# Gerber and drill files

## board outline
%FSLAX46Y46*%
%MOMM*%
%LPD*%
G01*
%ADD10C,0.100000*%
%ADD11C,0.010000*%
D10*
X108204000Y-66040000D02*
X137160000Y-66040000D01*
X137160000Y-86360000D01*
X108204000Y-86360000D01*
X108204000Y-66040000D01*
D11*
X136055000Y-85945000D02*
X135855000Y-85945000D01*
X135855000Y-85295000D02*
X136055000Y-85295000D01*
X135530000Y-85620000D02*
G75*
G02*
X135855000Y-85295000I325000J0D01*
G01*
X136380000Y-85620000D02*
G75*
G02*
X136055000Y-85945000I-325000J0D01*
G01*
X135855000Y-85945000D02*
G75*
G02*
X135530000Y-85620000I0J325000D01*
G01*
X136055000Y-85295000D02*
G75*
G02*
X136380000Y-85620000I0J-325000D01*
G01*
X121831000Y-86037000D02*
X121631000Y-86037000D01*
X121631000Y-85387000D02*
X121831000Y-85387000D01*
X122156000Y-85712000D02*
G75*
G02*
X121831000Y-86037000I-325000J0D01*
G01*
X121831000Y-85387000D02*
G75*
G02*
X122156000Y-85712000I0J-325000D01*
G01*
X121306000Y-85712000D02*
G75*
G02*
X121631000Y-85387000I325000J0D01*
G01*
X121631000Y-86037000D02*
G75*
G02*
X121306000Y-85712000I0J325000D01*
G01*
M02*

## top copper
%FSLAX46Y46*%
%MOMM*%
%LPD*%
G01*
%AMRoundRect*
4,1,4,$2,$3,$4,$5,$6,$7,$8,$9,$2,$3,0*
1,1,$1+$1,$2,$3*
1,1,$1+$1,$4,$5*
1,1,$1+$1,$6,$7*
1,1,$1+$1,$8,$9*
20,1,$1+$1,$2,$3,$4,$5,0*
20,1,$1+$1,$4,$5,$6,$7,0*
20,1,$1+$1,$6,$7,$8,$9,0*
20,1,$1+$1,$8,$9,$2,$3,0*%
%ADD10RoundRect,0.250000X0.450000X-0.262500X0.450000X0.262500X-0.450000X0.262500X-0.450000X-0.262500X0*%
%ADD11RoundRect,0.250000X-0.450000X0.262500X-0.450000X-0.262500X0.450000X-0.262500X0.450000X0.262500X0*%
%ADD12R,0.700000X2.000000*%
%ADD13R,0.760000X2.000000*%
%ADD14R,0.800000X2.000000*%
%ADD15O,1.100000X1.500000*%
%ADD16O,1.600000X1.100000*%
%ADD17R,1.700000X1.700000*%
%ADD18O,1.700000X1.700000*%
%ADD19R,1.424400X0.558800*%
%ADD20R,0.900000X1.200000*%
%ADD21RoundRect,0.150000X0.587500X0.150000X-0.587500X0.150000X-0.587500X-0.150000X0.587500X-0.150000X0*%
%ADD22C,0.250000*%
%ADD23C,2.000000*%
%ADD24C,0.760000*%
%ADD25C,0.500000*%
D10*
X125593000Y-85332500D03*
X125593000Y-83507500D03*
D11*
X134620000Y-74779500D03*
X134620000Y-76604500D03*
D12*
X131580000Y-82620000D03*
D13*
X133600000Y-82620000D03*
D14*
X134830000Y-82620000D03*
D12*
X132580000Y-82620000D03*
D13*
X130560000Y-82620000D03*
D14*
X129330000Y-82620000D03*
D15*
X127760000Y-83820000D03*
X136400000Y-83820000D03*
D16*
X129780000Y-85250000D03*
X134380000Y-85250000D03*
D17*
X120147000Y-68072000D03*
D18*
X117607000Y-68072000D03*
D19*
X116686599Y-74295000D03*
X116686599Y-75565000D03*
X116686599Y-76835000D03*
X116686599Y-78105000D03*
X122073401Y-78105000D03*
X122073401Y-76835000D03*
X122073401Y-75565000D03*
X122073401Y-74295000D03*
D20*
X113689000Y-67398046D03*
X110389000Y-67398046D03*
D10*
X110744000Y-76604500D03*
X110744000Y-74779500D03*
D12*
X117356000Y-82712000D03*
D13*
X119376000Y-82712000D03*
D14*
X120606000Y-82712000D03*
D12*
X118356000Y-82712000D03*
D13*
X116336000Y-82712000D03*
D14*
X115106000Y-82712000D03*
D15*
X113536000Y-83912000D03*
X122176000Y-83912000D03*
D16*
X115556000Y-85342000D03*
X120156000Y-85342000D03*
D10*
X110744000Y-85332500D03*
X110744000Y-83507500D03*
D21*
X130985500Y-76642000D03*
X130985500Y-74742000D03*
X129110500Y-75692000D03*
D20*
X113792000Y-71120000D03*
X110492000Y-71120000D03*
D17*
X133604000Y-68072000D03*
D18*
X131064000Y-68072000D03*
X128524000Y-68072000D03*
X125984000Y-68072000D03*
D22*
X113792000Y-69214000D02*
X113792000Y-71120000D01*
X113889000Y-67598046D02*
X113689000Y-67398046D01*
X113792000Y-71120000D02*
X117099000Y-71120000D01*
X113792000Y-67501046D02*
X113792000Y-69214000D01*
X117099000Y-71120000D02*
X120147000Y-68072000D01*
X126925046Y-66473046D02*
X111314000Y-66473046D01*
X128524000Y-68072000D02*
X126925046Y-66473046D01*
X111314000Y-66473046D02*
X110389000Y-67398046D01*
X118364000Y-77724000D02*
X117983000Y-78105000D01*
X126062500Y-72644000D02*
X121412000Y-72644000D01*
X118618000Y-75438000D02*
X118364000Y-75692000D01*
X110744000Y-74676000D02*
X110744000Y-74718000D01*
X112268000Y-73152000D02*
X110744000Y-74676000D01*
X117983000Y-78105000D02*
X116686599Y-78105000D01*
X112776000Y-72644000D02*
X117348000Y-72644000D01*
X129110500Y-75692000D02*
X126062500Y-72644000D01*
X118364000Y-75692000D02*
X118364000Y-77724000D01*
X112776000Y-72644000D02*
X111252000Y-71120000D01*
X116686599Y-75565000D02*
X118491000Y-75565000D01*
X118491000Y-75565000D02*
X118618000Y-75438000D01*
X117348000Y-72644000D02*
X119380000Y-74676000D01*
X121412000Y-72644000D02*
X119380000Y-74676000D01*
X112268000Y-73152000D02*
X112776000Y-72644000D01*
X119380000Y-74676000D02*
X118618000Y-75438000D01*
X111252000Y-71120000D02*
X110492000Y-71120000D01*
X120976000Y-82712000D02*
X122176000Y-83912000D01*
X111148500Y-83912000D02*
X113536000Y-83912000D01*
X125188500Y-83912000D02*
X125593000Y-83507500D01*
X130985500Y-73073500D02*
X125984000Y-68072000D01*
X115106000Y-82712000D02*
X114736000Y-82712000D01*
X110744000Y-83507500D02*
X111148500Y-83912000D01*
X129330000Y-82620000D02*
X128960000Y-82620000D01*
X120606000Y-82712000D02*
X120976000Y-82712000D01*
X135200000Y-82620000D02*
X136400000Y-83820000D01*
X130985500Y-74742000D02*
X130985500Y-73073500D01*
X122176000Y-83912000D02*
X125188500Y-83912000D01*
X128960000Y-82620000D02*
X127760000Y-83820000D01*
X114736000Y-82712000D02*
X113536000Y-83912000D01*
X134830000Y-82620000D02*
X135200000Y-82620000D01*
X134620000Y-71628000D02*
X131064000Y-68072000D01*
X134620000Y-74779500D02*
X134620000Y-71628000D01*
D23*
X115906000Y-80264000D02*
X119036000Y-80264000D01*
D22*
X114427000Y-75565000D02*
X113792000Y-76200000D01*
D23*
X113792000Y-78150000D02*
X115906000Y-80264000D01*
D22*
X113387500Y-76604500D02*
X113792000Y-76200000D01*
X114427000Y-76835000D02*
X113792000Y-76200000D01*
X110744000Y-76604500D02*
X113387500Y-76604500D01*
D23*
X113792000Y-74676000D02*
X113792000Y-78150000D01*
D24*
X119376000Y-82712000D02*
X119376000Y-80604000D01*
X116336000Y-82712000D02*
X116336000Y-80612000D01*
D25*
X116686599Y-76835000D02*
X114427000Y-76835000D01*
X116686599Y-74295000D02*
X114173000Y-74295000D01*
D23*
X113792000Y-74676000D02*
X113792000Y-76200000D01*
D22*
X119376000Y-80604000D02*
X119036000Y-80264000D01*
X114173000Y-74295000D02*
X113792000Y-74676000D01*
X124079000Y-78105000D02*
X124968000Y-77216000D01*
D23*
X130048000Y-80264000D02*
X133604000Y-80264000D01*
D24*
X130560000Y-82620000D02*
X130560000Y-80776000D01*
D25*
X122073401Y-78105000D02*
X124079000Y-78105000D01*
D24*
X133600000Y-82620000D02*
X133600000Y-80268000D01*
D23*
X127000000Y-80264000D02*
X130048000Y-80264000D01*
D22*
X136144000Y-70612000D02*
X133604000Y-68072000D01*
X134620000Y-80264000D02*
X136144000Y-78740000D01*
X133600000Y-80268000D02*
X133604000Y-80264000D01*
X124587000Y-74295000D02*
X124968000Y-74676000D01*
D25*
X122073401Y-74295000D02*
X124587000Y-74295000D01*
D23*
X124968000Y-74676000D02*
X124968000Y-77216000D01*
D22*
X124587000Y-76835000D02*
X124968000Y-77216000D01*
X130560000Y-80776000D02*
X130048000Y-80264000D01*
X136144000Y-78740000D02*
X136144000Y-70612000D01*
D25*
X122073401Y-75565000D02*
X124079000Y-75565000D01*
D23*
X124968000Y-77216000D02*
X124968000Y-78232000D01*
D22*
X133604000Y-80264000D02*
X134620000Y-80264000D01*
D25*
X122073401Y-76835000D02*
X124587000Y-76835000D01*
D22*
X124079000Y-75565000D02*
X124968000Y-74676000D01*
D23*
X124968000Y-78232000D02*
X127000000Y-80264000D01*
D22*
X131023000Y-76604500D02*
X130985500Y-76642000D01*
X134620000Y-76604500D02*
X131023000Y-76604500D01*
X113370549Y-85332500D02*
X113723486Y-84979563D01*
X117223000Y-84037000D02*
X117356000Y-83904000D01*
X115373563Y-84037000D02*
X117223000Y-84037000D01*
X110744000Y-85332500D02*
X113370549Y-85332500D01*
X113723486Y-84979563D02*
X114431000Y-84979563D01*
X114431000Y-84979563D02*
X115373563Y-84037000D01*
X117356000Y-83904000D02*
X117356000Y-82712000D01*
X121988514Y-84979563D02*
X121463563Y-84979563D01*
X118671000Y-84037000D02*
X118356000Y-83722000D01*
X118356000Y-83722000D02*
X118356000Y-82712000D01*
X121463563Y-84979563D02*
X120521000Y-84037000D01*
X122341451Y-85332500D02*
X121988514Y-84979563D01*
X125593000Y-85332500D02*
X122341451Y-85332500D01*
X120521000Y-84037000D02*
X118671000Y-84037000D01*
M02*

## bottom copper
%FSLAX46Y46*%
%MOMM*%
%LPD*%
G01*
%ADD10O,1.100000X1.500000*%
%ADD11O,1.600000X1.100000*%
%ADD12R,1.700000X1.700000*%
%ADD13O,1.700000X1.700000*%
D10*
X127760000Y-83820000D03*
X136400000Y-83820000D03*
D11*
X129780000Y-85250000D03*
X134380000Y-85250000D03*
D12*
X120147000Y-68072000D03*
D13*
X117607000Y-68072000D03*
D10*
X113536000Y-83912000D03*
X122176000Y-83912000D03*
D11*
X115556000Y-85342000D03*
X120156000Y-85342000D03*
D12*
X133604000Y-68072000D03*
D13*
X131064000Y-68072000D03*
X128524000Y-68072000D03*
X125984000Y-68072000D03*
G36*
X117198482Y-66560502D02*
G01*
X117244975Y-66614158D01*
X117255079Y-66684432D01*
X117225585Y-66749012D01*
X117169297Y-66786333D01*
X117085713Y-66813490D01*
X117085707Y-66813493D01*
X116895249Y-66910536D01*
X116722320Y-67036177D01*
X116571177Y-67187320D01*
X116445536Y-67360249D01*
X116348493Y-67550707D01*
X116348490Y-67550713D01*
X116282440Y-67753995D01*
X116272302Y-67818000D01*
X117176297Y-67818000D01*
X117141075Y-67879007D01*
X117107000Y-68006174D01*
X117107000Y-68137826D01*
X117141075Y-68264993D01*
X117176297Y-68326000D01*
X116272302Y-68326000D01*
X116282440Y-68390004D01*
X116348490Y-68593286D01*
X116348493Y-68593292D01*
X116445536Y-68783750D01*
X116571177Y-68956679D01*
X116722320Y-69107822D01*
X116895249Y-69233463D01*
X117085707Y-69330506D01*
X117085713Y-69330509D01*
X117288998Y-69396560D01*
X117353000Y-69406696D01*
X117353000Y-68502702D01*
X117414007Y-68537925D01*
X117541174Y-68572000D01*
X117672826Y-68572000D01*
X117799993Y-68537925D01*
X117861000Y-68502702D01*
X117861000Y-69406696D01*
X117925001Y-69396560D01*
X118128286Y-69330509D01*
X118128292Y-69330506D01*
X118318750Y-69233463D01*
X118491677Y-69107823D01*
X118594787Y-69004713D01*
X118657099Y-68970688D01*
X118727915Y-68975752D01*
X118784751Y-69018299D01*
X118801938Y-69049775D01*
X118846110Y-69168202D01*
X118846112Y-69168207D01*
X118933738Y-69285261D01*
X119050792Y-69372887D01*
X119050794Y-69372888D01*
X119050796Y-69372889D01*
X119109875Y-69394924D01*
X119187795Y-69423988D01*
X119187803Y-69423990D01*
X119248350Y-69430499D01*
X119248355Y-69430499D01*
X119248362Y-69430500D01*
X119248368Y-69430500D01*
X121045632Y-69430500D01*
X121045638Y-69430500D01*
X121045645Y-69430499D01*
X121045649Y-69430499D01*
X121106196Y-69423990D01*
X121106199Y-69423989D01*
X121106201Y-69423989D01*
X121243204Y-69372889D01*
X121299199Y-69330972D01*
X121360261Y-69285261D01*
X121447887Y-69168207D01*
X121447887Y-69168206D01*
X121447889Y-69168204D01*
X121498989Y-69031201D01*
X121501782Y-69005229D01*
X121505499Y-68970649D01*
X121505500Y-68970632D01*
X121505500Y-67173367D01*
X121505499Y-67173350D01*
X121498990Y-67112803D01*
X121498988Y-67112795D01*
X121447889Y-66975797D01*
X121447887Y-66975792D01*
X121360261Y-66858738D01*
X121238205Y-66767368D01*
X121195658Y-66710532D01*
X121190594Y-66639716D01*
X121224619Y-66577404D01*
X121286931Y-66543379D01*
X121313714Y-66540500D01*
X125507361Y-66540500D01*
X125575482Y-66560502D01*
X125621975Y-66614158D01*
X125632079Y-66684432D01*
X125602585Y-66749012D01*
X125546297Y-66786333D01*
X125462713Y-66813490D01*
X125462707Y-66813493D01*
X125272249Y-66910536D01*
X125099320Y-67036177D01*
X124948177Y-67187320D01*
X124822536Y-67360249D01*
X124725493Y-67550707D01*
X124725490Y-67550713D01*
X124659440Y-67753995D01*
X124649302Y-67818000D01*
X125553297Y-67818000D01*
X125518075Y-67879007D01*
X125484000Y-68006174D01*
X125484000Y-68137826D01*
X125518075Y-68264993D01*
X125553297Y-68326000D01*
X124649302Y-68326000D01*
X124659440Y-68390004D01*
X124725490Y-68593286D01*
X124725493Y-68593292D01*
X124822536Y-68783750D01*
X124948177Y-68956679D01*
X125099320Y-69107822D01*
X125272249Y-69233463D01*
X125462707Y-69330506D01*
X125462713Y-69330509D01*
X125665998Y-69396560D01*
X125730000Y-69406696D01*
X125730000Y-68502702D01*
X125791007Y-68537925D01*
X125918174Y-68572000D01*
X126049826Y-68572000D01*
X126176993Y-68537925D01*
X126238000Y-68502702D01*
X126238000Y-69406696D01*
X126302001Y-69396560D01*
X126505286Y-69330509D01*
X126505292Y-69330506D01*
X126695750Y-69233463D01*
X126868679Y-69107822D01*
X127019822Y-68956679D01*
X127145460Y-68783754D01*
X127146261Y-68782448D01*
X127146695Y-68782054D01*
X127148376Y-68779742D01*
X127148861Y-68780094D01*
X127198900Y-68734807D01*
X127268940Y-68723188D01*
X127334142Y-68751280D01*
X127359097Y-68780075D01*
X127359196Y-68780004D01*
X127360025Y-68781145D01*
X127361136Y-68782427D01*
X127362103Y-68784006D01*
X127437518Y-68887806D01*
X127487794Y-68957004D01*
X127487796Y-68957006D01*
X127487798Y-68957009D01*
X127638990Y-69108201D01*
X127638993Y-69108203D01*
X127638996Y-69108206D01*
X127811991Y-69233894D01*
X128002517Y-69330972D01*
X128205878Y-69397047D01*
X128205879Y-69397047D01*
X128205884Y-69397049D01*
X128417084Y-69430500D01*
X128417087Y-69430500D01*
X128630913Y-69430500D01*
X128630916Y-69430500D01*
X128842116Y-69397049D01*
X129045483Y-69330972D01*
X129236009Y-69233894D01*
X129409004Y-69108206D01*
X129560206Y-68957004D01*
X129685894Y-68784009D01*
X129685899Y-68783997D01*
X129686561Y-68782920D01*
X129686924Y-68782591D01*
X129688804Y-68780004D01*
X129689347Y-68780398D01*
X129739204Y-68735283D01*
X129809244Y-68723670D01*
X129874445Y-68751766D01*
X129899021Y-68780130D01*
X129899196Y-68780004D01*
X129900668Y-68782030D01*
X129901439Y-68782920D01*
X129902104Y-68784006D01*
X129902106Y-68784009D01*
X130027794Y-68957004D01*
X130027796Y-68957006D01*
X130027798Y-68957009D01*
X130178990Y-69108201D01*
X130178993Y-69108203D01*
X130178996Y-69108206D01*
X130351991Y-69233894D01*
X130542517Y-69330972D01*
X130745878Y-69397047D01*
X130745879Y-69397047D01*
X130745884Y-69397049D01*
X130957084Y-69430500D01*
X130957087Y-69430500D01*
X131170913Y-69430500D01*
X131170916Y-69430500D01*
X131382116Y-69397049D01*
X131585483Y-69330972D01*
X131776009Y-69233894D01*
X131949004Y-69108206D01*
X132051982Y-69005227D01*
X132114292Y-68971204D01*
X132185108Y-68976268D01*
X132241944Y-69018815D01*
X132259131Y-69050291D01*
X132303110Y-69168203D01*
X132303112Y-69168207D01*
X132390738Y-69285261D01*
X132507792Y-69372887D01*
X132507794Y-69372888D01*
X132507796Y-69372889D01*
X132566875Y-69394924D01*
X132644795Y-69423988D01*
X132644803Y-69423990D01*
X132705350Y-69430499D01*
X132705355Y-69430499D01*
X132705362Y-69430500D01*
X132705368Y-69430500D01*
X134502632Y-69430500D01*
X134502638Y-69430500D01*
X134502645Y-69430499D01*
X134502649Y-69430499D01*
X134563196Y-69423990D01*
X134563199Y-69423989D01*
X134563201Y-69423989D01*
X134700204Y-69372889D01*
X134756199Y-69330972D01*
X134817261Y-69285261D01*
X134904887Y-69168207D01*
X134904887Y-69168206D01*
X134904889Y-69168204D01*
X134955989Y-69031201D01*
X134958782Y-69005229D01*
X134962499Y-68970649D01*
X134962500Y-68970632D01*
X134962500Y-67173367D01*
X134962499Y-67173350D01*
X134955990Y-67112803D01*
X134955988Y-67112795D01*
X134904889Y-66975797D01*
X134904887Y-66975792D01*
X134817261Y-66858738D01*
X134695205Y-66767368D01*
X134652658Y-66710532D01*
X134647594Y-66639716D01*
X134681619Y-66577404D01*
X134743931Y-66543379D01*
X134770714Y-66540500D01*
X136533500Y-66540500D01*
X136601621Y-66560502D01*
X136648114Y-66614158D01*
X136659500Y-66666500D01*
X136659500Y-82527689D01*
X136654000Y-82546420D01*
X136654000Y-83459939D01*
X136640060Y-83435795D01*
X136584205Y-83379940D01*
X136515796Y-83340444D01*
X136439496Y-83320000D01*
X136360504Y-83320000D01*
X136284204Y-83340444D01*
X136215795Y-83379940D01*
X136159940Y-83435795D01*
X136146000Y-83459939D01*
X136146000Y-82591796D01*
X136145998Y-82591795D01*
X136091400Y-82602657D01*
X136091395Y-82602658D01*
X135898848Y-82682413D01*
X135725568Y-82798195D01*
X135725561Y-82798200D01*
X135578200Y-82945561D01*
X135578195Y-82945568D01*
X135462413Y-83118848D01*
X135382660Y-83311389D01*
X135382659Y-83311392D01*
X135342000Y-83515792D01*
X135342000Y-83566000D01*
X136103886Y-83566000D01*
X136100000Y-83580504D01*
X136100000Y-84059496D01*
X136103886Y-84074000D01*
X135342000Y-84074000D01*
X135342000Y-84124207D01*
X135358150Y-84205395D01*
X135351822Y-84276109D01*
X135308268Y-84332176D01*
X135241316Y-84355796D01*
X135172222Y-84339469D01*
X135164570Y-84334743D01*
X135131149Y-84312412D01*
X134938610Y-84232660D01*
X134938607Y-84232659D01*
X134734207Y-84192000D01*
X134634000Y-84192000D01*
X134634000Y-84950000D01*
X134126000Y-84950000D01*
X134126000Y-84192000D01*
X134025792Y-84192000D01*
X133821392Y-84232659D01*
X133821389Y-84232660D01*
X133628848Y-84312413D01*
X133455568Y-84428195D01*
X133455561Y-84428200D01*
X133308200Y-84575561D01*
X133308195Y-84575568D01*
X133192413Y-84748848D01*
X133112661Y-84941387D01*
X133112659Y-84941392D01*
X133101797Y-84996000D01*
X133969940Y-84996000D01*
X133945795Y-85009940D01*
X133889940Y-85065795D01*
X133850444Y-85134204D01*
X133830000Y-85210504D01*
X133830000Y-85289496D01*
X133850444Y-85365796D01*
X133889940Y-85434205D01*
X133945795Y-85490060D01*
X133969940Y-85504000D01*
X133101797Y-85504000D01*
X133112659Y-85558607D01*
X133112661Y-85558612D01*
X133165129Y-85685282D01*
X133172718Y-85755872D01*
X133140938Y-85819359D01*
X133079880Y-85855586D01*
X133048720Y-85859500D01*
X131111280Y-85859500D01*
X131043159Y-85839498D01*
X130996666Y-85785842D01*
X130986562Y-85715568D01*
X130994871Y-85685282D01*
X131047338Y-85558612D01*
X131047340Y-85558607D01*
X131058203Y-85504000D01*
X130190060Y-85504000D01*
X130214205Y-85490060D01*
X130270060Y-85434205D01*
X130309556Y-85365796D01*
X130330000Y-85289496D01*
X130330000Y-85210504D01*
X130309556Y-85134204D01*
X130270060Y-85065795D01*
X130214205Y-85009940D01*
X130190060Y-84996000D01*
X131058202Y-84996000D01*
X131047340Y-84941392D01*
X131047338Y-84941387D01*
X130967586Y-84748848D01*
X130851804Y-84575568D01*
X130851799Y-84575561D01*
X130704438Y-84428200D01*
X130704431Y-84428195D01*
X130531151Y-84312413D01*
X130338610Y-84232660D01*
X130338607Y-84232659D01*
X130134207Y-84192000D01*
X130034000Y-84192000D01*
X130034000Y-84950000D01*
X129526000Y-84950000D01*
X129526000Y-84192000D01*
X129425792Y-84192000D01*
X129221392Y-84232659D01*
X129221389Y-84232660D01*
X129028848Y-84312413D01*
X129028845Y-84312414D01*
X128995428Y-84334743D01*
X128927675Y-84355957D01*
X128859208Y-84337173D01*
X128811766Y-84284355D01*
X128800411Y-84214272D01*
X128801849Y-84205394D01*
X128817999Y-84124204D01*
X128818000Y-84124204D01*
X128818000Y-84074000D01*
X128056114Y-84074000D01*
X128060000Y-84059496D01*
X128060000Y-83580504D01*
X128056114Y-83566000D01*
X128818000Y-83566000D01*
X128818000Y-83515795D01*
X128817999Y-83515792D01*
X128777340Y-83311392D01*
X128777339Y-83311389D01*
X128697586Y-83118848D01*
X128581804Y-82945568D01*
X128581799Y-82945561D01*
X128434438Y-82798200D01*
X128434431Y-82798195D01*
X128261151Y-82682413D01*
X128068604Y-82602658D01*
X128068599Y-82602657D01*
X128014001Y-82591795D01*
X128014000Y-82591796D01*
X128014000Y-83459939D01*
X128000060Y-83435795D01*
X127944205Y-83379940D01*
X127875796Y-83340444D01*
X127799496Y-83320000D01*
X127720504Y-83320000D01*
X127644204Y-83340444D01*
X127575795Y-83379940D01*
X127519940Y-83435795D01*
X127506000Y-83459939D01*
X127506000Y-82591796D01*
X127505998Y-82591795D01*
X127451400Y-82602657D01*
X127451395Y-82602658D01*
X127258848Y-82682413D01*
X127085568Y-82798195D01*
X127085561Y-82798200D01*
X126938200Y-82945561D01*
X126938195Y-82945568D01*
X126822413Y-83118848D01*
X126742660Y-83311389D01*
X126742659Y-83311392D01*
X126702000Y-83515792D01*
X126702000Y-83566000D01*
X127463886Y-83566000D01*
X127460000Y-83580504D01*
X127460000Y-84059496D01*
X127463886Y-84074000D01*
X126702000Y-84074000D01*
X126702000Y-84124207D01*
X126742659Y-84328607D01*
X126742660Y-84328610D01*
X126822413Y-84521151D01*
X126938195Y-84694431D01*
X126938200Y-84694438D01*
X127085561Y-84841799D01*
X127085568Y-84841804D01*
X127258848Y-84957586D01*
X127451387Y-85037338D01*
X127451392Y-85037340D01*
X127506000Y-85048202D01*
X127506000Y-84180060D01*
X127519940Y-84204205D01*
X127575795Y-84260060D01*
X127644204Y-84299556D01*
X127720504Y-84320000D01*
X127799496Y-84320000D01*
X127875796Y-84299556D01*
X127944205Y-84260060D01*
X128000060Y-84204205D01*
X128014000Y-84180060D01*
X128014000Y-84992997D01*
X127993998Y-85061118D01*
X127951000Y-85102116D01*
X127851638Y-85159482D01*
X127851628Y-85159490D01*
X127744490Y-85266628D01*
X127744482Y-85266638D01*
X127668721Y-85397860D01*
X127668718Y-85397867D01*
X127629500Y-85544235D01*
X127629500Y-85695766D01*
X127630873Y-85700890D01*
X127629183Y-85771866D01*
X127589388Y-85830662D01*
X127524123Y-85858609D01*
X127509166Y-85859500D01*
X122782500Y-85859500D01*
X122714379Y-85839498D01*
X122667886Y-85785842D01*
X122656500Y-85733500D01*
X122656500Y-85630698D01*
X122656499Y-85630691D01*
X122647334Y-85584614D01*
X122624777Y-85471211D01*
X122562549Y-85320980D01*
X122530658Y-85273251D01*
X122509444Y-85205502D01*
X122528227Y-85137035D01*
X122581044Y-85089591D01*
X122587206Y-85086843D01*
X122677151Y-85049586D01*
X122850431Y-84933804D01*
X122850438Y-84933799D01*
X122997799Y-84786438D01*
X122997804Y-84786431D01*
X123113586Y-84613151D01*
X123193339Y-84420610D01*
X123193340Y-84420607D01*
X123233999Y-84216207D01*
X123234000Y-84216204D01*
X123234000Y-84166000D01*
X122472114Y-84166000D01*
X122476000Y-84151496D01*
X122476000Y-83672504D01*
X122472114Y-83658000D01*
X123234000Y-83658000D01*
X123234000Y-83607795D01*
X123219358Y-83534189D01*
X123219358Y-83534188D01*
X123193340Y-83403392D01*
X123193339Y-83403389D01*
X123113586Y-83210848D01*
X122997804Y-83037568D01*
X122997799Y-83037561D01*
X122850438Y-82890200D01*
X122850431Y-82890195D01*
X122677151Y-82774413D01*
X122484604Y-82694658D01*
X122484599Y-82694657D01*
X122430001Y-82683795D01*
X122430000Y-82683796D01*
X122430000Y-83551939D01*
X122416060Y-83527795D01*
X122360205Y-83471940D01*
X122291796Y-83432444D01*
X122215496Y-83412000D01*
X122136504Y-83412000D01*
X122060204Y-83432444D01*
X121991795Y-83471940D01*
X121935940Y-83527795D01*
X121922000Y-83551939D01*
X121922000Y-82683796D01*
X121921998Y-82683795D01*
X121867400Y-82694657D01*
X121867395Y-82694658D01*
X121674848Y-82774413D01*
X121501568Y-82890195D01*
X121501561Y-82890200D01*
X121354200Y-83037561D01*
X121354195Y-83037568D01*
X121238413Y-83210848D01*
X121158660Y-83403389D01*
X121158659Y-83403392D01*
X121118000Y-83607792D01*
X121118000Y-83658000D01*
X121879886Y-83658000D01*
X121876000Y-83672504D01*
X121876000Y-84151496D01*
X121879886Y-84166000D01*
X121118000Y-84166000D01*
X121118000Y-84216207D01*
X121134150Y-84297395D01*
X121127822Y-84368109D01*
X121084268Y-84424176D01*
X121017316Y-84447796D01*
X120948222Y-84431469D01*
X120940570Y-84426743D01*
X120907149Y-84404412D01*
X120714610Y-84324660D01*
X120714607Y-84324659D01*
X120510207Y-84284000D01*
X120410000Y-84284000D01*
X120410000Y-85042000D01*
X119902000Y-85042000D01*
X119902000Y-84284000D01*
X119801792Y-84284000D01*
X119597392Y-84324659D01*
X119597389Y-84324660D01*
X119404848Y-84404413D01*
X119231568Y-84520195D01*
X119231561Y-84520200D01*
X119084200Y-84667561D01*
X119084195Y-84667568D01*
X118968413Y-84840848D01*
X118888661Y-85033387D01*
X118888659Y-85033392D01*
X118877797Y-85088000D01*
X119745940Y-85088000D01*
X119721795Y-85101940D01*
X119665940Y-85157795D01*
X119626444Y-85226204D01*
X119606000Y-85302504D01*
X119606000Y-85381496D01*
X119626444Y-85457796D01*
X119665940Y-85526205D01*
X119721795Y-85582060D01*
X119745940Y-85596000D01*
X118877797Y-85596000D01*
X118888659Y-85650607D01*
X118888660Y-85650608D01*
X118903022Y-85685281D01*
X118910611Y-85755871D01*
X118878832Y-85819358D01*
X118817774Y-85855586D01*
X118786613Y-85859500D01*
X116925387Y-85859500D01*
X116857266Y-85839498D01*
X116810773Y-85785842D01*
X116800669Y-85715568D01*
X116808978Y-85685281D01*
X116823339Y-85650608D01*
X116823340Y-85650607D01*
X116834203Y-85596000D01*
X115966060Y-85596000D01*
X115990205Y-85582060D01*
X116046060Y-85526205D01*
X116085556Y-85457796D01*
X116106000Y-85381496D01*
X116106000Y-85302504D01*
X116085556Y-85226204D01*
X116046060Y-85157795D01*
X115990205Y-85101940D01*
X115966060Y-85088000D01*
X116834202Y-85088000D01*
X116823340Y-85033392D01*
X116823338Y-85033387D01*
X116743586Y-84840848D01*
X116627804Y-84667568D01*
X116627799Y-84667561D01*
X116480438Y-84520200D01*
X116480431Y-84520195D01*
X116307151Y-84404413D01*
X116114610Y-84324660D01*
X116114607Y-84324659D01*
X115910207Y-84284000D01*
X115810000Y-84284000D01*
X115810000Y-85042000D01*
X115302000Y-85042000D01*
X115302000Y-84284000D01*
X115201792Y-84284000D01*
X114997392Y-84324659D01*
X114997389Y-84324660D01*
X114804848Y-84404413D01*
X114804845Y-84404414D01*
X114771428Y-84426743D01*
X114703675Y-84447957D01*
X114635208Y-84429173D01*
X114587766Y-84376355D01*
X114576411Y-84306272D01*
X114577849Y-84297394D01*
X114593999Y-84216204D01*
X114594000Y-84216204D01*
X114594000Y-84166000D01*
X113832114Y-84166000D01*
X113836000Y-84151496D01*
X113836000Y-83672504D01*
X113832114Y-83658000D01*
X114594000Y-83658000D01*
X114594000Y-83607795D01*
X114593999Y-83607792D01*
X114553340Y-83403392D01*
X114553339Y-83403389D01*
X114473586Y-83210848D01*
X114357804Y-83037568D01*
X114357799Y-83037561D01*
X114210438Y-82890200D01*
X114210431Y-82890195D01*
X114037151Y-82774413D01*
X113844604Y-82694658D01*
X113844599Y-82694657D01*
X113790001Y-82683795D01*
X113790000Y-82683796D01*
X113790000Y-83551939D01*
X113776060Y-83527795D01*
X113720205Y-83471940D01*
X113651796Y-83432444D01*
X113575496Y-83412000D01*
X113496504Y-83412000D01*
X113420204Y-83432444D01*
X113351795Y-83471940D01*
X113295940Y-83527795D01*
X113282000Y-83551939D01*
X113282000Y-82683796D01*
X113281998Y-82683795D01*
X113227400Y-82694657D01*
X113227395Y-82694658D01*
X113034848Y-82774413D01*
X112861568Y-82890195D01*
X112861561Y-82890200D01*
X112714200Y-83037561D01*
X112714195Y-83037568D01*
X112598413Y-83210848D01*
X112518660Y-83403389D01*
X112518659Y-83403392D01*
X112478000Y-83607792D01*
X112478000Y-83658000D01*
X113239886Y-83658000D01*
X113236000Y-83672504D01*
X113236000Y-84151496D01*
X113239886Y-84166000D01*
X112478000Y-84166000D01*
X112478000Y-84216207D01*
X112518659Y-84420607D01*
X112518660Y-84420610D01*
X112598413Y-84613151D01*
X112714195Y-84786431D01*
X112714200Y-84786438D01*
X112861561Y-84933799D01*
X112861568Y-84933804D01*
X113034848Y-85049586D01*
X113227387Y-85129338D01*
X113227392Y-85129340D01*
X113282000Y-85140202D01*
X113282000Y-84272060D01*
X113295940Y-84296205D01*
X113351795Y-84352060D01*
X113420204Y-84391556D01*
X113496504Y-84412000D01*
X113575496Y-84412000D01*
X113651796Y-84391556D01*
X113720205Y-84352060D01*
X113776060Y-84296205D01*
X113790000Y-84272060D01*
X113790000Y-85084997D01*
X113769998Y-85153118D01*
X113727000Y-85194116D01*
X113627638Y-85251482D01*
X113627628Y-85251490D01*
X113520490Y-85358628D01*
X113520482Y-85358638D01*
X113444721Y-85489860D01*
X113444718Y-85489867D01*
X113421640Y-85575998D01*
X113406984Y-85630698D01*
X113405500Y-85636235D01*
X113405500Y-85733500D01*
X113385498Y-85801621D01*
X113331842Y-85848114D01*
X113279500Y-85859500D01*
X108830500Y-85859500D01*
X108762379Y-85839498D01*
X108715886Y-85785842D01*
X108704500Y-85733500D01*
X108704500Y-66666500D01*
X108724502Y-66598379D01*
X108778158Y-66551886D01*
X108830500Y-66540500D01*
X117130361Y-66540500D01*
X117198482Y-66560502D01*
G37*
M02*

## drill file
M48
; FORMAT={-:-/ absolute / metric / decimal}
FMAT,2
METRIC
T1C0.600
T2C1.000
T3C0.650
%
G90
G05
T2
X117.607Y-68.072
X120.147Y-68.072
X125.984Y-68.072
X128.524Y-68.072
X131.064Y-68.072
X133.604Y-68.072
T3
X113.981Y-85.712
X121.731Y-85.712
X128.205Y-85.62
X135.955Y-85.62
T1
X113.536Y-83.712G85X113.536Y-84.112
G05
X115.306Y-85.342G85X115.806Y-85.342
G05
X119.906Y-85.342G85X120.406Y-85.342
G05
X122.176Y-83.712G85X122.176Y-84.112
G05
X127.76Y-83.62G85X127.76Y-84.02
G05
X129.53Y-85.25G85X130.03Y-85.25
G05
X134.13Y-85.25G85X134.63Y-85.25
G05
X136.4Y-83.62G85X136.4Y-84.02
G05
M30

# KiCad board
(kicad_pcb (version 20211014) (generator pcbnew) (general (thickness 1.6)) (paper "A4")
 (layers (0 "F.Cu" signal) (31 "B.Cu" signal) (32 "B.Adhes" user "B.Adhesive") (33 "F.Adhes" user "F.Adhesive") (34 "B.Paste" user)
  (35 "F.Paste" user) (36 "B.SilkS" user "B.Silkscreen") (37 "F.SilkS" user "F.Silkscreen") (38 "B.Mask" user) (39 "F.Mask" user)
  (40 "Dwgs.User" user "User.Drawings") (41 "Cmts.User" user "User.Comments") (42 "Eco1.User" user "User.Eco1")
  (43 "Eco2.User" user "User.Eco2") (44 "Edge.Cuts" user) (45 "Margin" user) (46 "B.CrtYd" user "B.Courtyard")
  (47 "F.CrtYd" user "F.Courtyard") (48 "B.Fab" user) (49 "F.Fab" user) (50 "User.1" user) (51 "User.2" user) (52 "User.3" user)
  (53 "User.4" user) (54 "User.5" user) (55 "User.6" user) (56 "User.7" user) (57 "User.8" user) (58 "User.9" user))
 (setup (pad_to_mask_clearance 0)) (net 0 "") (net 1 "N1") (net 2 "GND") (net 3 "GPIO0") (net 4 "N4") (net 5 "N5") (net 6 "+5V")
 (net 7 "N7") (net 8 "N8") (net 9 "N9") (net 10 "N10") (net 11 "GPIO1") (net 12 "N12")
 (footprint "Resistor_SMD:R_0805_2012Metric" (layer "F.Cu") (at 125.593 84.42 90)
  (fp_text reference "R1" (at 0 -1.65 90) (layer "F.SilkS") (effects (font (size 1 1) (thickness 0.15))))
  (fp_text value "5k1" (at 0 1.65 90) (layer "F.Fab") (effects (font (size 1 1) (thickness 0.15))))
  (pad "1" smd roundrect (at -0.9125 0 90) (size 1.025 1.4) (layers "F.Cu" "F.Paste" "F.Mask") (roundrect_rratio 0.243902) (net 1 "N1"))
  (pad "2" smd roundrect (at 0.9125 0 90) (size 1.025 1.4) (layers "F.Cu" "F.Paste" "F.Mask") (roundrect_rratio 0.243902) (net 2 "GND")))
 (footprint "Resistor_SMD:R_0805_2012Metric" (layer "F.Cu") (at 134.62 75.692 -90)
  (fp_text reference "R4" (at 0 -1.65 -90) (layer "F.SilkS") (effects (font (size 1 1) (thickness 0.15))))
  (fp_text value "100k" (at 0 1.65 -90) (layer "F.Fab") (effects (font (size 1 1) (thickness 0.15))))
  (pad "1" smd roundrect (at -0.9125 0 270) (size 1.025 1.4) (layers "F.Cu" "F.Paste" "F.Mask") (roundrect_rratio 0.243902) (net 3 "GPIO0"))
  (pad "2" smd roundrect (at 0.9125 0 270) (size 1.025 1.4) (layers "F.Cu" "F.Paste" "F.Mask") (roundrect_rratio 0.243902) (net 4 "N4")))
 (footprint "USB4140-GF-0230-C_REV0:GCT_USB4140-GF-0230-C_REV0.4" (layer "F.Cu") (at 132.08 83.82)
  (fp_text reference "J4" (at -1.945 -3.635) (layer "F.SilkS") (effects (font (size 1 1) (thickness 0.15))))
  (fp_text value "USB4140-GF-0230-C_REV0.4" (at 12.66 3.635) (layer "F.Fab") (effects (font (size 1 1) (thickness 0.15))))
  (fp_line (start 3.975 2.125) (end 3.775 2.125) (layer "Edge.Cuts") (width 0.01))
  (fp_line (start 3.775 1.475) (end 3.975 1.475) (layer "Edge.Cuts") (width 0.01))
  (fp_arc (start 3.45 1.8) (mid 3.54519 1.57019) (end 3.775 1.475) (layer "Edge.Cuts") (width 0.01))
  (fp_arc (start 4.3 1.8) (mid 4.20481 2.02981) (end 3.975 2.125) (layer "Edge.Cuts") (width 0.01))
  (fp_arc (start 3.775 2.125) (mid 3.54519 2.02981) (end 3.45 1.8) (layer "Edge.Cuts") (width 0.01))
  (fp_arc (start 3.975 1.475) (mid 4.20481 1.57019) (end 4.3 1.8) (layer "Edge.Cuts") (width 0.01))
  (pad "" np_thru_hole circle locked (at 3.875 1.8) (size 0.65 0.65) (drill 0.65) (layers *.Cu *.Mask))
  (pad "" np_thru_hole circle locked (at -3.875 1.8) (size 0.65 0.65) (drill 0.65) (layers *.Cu *.Mask))
  (pad "A5" smd rect locked (at -0.5 -1.2) (size 0.7 2) (layers "F.Cu" "F.Paste" "F.Mask") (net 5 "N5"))
  (pad "A9" smd rect locked (at 1.52 -1.2) (size 0.76 2) (layers "F.Cu" "F.Paste" "F.Mask") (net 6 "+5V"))
  (pad "A12" smd rect locked (at 2.75 -1.2) (size 0.8 2) (layers "F.Cu" "F.Paste" "F.Mask") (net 2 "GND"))
  (pad "B5" smd rect locked (at 0.5 -1.2) (size 0.7 2) (layers "F.Cu" "F.Paste" "F.Mask") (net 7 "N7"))
  (pad "B9" smd rect locked (at -1.52 -1.2) (size 0.76 2) (layers "F.Cu" "F.Paste" "F.Mask") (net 6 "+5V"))
  (pad "B12" smd rect locked (at -2.75 -1.2) (size 0.8 2) (layers "F.Cu" "F.Paste" "F.Mask") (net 2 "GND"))
  (pad "S1" thru_hole oval locked (at -4.32 0) (size 1.1 1.5) (drill oval 0.6 1) (layers *.Cu *.Mask) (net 2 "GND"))
  (pad "S2" thru_hole oval locked (at 4.32 0) (size 1.1 1.5) (drill oval 0.6 1) (layers *.Cu *.Mask) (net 2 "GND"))
  (pad "S3" thru_hole oval locked (at -2.3 1.43) (size 1.6 1.1) (drill oval 1.1 0.6) (layers *.Cu *.Mask) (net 2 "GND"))
  (pad "S4" thru_hole oval locked (at 2.3 1.43) (size 1.6 1.1) (drill oval 1.1 0.6) (layers *.Cu *.Mask) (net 2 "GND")))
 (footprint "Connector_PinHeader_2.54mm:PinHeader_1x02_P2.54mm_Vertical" (layer "F.Cu") (at 120.147 68.072 -90)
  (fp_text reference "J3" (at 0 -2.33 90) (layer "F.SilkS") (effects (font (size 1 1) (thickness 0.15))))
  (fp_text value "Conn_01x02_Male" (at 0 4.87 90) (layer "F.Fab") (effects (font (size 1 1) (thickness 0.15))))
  (pad "1" thru_hole rect (at 0 0 270) (size 1.7 1.7) (drill 1) (layers *.Cu *.Mask) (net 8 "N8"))
  (pad "2" thru_hole oval (at 0 2.54 270) (size 1.7 1.7) (drill 1) (layers *.Cu *.Mask) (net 2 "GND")))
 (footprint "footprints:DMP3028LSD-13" (layer "F.Cu") (at 119.38 76.2)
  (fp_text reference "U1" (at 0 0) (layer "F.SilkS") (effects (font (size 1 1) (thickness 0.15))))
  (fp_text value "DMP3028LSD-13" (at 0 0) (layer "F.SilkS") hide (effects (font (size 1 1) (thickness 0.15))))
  (pad "1" smd rect (at -2.693401 -1.905) (size 1.4244 0.5588) (layers "F.Cu" "F.Paste" "F.Mask") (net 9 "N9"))
  (pad "2" smd rect (at -2.693401 -0.635) (size 1.4244 0.5588) (layers "F.Cu" "F.Paste" "F.Mask") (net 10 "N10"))
  (pad "3" smd rect (at -2.693401 0.635) (size 1.4244 0.5588) (layers "F.Cu" "F.Paste" "F.Mask") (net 9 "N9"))
  (pad "4" smd rect (at -2.693401 1.905) (size 1.4244 0.5588) (layers "F.Cu" "F.Paste" "F.Mask") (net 10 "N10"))
  (pad "5" smd rect (at 2.693401 1.905) (size 1.4244 0.5588) (layers "F.Cu" "F.Paste" "F.Mask") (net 6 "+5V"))
  (pad "6" smd rect (at 2.693401 0.635) (size 1.4244 0.5588) (layers "F.Cu" "F.Paste" "F.Mask") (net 6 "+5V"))
  (pad "7" smd rect (at 2.693401 -0.635) (size 1.4244 0.5588) (layers "F.Cu" "F.Paste" "F.Mask") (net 6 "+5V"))
  (pad "8" smd rect (at 2.693401 -1.905) (size 1.4244 0.5588) (layers "F.Cu" "F.Paste" "F.Mask") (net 6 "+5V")))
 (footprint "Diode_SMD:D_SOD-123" (layer "F.Cu") (at 112.039 67.398046 180)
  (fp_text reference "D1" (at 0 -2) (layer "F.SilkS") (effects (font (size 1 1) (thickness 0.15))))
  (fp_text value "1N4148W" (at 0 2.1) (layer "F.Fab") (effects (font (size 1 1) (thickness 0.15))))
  (pad "1" smd rect (at -1.65 0 180) (size 0.9 1.2) (layers "F.Cu" "F.Paste" "F.Mask") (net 8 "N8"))
  (pad "2" smd rect (at 1.65 0 180) (size 0.9 1.2) (layers "F.Cu" "F.Paste" "F.Mask") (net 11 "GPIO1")))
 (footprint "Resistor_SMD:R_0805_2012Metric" (layer "F.Cu") (at 110.744 75.692 90)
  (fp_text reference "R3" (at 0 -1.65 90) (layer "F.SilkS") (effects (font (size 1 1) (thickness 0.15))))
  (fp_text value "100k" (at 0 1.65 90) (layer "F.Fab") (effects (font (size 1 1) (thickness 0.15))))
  (pad "1" smd roundrect (at -0.9125 0 90) (size 1.025 1.4) (layers "F.Cu" "F.Paste" "F.Mask") (roundrect_rratio 0.243902) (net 9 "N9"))
  (pad "2" smd roundrect (at 0.9125 0 90) (size 1.025 1.4) (layers "F.Cu" "F.Paste" "F.Mask") (roundrect_rratio 0.243902) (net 10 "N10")))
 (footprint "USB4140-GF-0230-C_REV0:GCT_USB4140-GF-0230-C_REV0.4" (layer "F.Cu") (at 117.856 83.912)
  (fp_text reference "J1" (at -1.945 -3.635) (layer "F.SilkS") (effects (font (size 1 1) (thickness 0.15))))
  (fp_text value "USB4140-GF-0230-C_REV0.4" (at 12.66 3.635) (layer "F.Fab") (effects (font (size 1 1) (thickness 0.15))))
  (fp_line (start 3.975 2.125) (end 3.775 2.125) (layer "Edge.Cuts") (width 0.01))
  (fp_line (start 3.775 1.475) (end 3.975 1.475) (layer "Edge.Cuts") (width 0.01))
  (fp_arc (start 4.3 1.8) (mid 4.20481 2.02981) (end 3.975 2.125) (layer "Edge.Cuts") (width 0.01))
  (fp_arc (start 3.975 1.475) (mid 4.20481 1.57019) (end 4.3 1.8) (layer "Edge.Cuts") (width 0.01))
  (fp_arc (start 3.45 1.8) (mid 3.54519 1.57019) (end 3.775 1.475) (layer "Edge.Cuts") (width 0.01))
  (fp_arc (start 3.775 2.125) (mid 3.54519 2.02981) (end 3.45 1.8) (layer "Edge.Cuts") (width 0.01))
  (pad "" np_thru_hole circle locked (at -3.875 1.8) (size 0.65 0.65) (drill 0.65) (layers *.Cu *.Mask))
  (pad "" np_thru_hole circle locked (at 3.875 1.8) (size 0.65 0.65) (drill 0.65) (layers *.Cu *.Mask))
  (pad "A5" smd rect locked (at -0.5 -1.2) (size 0.7 2) (layers "F.Cu" "F.Paste" "F.Mask") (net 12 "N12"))
  (pad "A9" smd rect locked (at 1.52 -1.2) (size 0.76 2) (layers "F.Cu" "F.Paste" "F.Mask") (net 9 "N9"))
  (pad "A12" smd rect locked (at 2.75 -1.2) (size 0.8 2) (layers "F.Cu" "F.Paste" "F.Mask") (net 2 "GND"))
  (pad "B5" smd rect locked (at 0.5 -1.2) (size 0.7 2) (layers "F.Cu" "F.Paste" "F.Mask") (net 1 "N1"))
  (pad "B9" smd rect locked (at -1.52 -1.2) (size 0.76 2) (layers "F.Cu" "F.Paste" "F.Mask") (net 9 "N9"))
  (pad "B12" smd rect locked (at -2.75 -1.2) (size 0.8 2) (layers "F.Cu" "F.Paste" "F.Mask") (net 2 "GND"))
  (pad "S1" thru_hole oval locked (at -4.32 0) (size 1.1 1.5) (drill oval 0.6 1) (layers *.Cu *.Mask) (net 2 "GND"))
  (pad "S2" thru_hole oval locked (at 4.32 0) (size 1.1 1.5) (drill oval 0.6 1) (layers *.Cu *.Mask) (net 2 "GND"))
  (pad "S3" thru_hole oval locked (at -2.3 1.43) (size 1.6 1.1) (drill oval 1.1 0.6) (layers *.Cu *.Mask) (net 2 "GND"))
  (pad "S4" thru_hole oval locked (at 2.3 1.43) (size 1.6 1.1) (drill oval 1.1 0.6) (layers *.Cu *.Mask) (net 2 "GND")))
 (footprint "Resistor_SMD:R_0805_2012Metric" (layer "F.Cu") (at 110.744 84.42 90)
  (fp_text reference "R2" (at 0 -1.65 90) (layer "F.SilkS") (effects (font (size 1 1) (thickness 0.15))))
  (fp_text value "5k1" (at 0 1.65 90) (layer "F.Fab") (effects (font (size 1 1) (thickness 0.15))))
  (pad "1" smd roundrect (at -0.9125 0 90) (size 1.025 1.4) (layers "F.Cu" "F.Paste" "F.Mask") (roundrect_rratio 0.243902) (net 12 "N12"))
  (pad "2" smd roundrect (at 0.9125 0 90) (size 1.025 1.4) (layers "F.Cu" "F.Paste" "F.Mask") (roundrect_rratio 0.243902) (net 2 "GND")))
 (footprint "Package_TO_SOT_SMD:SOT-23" (layer "F.Cu") (at 130.048 75.692 180)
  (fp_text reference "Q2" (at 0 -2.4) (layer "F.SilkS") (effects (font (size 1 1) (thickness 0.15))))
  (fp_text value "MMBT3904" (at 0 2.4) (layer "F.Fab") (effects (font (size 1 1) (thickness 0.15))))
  (pad "1" smd roundrect (at -0.9375 -0.95 180) (size 1.475 0.6) (layers "F.Cu" "F.Paste" "F.Mask") (roundrect_rratio 0.25) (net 4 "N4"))
  (pad "2" smd roundrect (at -0.9375 0.95 180) (size 1.475 0.6) (layers "F.Cu" "F.Paste" "F.Mask") (roundrect_rratio 0.25) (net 2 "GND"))
  (pad "3" smd roundrect (at 0.9375 0 180) (size 1.475 0.6) (layers "F.Cu" "F.Paste" "F.Mask") (roundrect_rratio 0.25) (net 10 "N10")))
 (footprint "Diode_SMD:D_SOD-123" (layer "F.Cu") (at 112.142 71.12 180)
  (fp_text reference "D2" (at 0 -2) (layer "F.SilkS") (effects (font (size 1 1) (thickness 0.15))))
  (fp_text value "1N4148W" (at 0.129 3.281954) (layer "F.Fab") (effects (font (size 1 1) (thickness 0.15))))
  (pad "1" smd rect (at -1.65 0 180) (size 0.9 1.2) (layers "F.Cu" "F.Paste" "F.Mask") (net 8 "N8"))
  (pad "2" smd rect (at 1.65 0 180) (size 0.9 1.2) (layers "F.Cu" "F.Paste" "F.Mask") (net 10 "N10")))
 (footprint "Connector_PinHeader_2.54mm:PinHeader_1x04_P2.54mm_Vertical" (layer "F.Cu") (at 133.604 68.072 -90)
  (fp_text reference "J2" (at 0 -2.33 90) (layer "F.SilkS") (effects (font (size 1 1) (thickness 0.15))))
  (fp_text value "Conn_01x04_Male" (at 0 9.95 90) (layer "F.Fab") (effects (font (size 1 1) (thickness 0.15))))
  (pad "1" thru_hole rect (at 0 0 270) (size 1.7 1.7) (drill 1) (layers *.Cu *.Mask) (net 6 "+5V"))
  (pad "2" thru_hole oval (at 0 2.54 270) (size 1.7 1.7) (drill 1) (layers *.Cu *.Mask) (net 3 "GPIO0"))
  (pad "3" thru_hole oval (at 0 5.08 270) (size 1.7 1.7) (drill 1) (layers *.Cu *.Mask) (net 11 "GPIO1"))
  (pad "4" thru_hole oval (at 0 7.62 270) (size 1.7 1.7) (drill 1) (layers *.Cu *.Mask) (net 2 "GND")))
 (gr_rect (start 108.204 66.04) (end 137.16 86.36) (layer "Edge.Cuts") (width 0.1) (fill none))
 (segment (start 113.792 69.214) (end 113.792 71.12) (width 0.25) (layer "F.Cu") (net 8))
 (segment (start 113.889 67.598046) (end 113.689 67.398046) (width 0.25) (layer "F.Cu") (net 8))
 (segment (start 113.792 71.12) (end 117.099 71.12) (width 0.25) (layer "F.Cu") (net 8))
 (segment (start 113.792 67.501046) (end 113.792 69.214) (width 0.25) (layer "F.Cu") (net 8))
 (segment (start 117.099 71.12) (end 120.147 68.072) (width 0.25) (layer "F.Cu") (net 8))
 (segment (start 126.925046 66.473046) (end 111.314 66.473046) (width 0.25) (layer "F.Cu") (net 11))
 (segment (start 128.524 68.072) (end 126.925046 66.473046) (width 0.25) (layer "F.Cu") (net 11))
 (segment (start 111.314 66.473046) (end 110.389 67.398046) (width 0.25) (layer "F.Cu") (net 11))
 (segment (start 118.364 77.724) (end 117.983 78.105) (width 0.25) (layer "F.Cu") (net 10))
 (segment (start 126.0625 72.644) (end 121.412 72.644) (width 0.25) (layer "F.Cu") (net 10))
 (segment (start 118.618 75.438) (end 118.364 75.692) (width 0.25) (layer "F.Cu") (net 10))
 (segment (start 110.744 74.676) (end 110.744 74.718) (width 0.25) (layer "F.Cu") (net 10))
 (segment (start 112.268 73.152) (end 110.744 74.676) (width 0.25) (layer "F.Cu") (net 10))
 (segment (start 117.983 78.105) (end 116.686599 78.105) (width 0.25) (layer "F.Cu") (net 10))
 (segment (start 112.776 72.644) (end 117.348 72.644) (width 0.25) (layer "F.Cu") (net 10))
 (segment (start 129.1105 75.692) (end 126.0625 72.644) (width 0.25) (layer "F.Cu") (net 10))
 (segment (start 118.364 75.692) (end 118.364 77.724) (width 0.25) (layer "F.Cu") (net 10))
 (segment (start 112.776 72.644) (end 111.252 71.12) (width 0.25) (layer "F.Cu") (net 10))
 (segment (start 116.686599 75.565) (end 118.491 75.565) (width 0.25) (layer "F.Cu") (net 10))
 (segment (start 118.491 75.565) (end 118.618 75.438) (width 0.25) (layer "F.Cu") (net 10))
 (segment (start 117.348 72.644) (end 119.38 74.676) (width 0.25) (layer "F.Cu") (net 10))
 (segment (start 121.412 72.644) (end 119.38 74.676) (width 0.25) (layer "F.Cu") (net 10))
 (segment (start 112.268 73.152) (end 112.776 72.644) (width 0.25) (layer "F.Cu") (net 10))
 (segment (start 119.38 74.676) (end 118.618 75.438) (width 0.25) (layer "F.Cu") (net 10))
 (segment (start 111.252 71.12) (end 110.492 71.12) (width 0.25) (layer "F.Cu") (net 10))
 (segment (start 120.976 82.712) (end 122.176 83.912) (width 0.25) (layer "F.Cu") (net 2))
 (segment (start 111.1485 83.912) (end 113.536 83.912) (width 0.25) (layer "F.Cu") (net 2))
 (segment (start 125.1885 83.912) (end 125.593 83.5075) (width 0.25) (layer "F.Cu") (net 2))
 (segment (start 130.9855 73.0735) (end 125.984 68.072) (width 0.25) (layer "F.Cu") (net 2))
 (segment (start 115.106 82.712) (end 114.736 82.712) (width 0.25) (layer "F.Cu") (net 2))
 (segment (start 110.744 83.5075) (end 111.1485 83.912) (width 0.25) (layer "F.Cu") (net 2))
 (segment (start 129.33 82.62) (end 128.96 82.62) (width 0.25) (layer "F.Cu") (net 2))
 (segment (start 120.606 82.712) (end 120.976 82.712) (width 0.25) (layer "F.Cu") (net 2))
 (segment (start 135.2 82.62) (end 136.4 83.82) (width 0.25) (layer "F.Cu") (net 2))
 (segment (start 130.9855 74.742) (end 130.9855 73.0735) (width 0.25) (layer "F.Cu") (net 2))
 (segment (start 122.176 83.912) (end 125.1885 83.912) (width 0.25) (layer "F.Cu") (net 2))
 (segment (start 128.96 82.62) (end 127.76 83.82) (width 0.25) (layer "F.Cu") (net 2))
 (segment (start 114.736 82.712) (end 113.536 83.912) (width 0.25) (layer "F.Cu") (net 2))
 (segment (start 134.83 82.62) (end 135.2 82.62) (width 0.25) (layer "F.Cu") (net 2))
 (segment (start 134.62 71.628) (end 131.064 68.072) (width 0.25) (layer "F.Cu") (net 3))
 (segment (start 134.62 74.7795) (end 134.62 71.628) (width 0.25) (layer "F.Cu") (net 3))
 (segment (start 115.906 80.264) (end 119.036 80.264) (width 2) (layer "F.Cu") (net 9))
 (segment (start 114.427 75.565) (end 113.792 76.2) (width 0.25) (layer "F.Cu") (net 9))
 (segment (start 113.792 78.15) (end 115.906 80.264) (width 2) (layer "F.Cu") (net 9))
 (segment (start 113.3875 76.6045) (end 113.792 76.2) (width 0.25) (layer "F.Cu") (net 9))
 (segment (start 114.427 76.835) (end 113.792 76.2) (width 0.25) (layer "F.Cu") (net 9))
 (segment (start 110.744 76.6045) (end 113.3875 76.6045) (width 0.25) (layer "F.Cu") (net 9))
 (segment (start 113.792 74.676) (end 113.792 78.15) (width 2) (layer "F.Cu") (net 9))
 (segment (start 119.376 82.712) (end 119.376 80.604) (width 0.76) (layer "F.Cu") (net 9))
 (segment (start 116.336 82.712) (end 116.336 80.612) (width 0.76) (layer "F.Cu") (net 9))
 (segment (start 116.686599 76.835) (end 114.427 76.835) (width 0.5) (layer "F.Cu") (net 9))
 (segment (start 116.686599 74.295) (end 114.173 74.295) (width 0.5) (layer "F.Cu") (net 9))
 (segment (start 113.792 74.676) (end 113.792 76.2) (width 2) (layer "F.Cu") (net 9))
 (segment (start 119.376 80.604) (end 119.036 80.264) (width 0.25) (layer "F.Cu") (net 9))
 (segment (start 114.173 74.295) (end 113.792 74.676) (width 0.25) (layer "F.Cu") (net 9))
 (segment (start 124.079 78.105) (end 124.968 77.216) (width 0.25) (layer "F.Cu") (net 6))
 (segment (start 130.048 80.264) (end 133.604 80.264) (width 2) (layer "F.Cu") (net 6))
 (segment (start 130.56 82.62) (end 130.56 80.776) (width 0.76) (layer "F.Cu") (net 6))
 (segment (start 122.073401 78.105) (end 124.079 78.105) (width 0.5) (layer "F.Cu") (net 6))
 (segment (start 133.6 82.62) (end 133.6 80.268) (width 0.76) (layer "F.Cu") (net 6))
 (segment (start 127 80.264) (end 130.048 80.264) (width 2) (layer "F.Cu") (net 6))
 (segment (start 136.144 70.612) (end 133.604 68.072) (width 0.25) (layer "F.Cu") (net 6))
 (segment (start 134.62 80.264) (end 136.144 78.74) (width 0.25) (layer "F.Cu") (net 6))
 (segment (start 133.6 80.268) (end 133.604 80.264) (width 0.25) (layer "F.Cu") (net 6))
 (segment (start 124.587 74.295) (end 124.968 74.676) (width 0.25) (layer "F.Cu") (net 6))
 (segment (start 122.073401 74.295) (end 124.587 74.295) (width 0.5) (layer "F.Cu") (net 6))
 (segment (start 124.968 74.676) (end 124.968 77.216) (width 2) (layer "F.Cu") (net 6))
 (segment (start 124.587 76.835) (end 124.968 77.216) (width 0.25) (layer "F.Cu") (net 6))
 (segment (start 130.56 80.776) (end 130.048 80.264) (width 0.25) (layer "F.Cu") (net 6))
 (segment (start 136.144 78.74) (end 136.144 70.612) (width 0.25) (layer "F.Cu") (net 6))
 (segment (start 122.073401 75.565) (end 124.079 75.565) (width 0.5) (layer "F.Cu") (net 6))
 (segment (start 124.968 77.216) (end 124.968 78.232) (width 2) (layer "F.Cu") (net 6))
 (segment (start 133.604 80.264) (end 134.62 80.264) (width 0.25) (layer "F.Cu") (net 6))
 (segment (start 122.073401 76.835) (end 124.587 76.835) (width 0.5) (layer "F.Cu") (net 6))
 (segment (start 124.079 75.565) (end 124.968 74.676) (width 0.25) (layer "F.Cu") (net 6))
 (segment (start 124.968 78.232) (end 127 80.264) (width 2) (layer "F.Cu") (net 6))
 (segment (start 131.023 76.6045) (end 130.9855 76.642) (width 0.25) (layer "F.Cu") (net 4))
 (segment (start 134.62 76.6045) (end 131.023 76.6045) (width 0.25) (layer "F.Cu") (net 4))
 (segment (start 113.370549 85.3325) (end 113.723486 84.979563) (width 0.25) (layer "F.Cu") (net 12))
 (segment (start 117.223 84.037) (end 117.356 83.904) (width 0.25) (layer "F.Cu") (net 12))
 (segment (start 115.373563 84.037) (end 117.223 84.037) (width 0.25) (layer "F.Cu") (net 12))
 (segment (start 110.744 85.3325) (end 113.370549 85.3325) (width 0.25) (layer "F.Cu") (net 12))
 (segment (start 113.723486 84.979563) (end 114.431 84.979563) (width 0.25) (layer "F.Cu") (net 12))
 (segment (start 114.431 84.979563) (end 115.373563 84.037) (width 0.25) (layer "F.Cu") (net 12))
 (segment (start 117.356 83.904) (end 117.356 82.712) (width 0.25) (layer "F.Cu") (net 12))
 (segment (start 121.988514 84.979563) (end 121.463563 84.979563) (width 0.25) (layer "F.Cu") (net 1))
 (segment (start 118.671 84.037) (end 118.356 83.722) (width 0.25) (layer "F.Cu") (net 1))
 (segment (start 118.356 83.722) (end 118.356 82.712) (width 0.25) (layer "F.Cu") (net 1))
 (segment (start 121.463563 84.979563) (end 120.521 84.037) (width 0.25) (layer "F.Cu") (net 1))
 (segment (start 122.341451 85.3325) (end 121.988514 84.979563) (width 0.25) (layer "F.Cu") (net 1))
 (segment (start 125.593 85.3325) (end 122.341451 85.3325) (width 0.25) (layer "F.Cu") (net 1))
 (segment (start 120.521 84.037) (end 118.671 84.037) (width 0.25) (layer "F.Cu") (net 1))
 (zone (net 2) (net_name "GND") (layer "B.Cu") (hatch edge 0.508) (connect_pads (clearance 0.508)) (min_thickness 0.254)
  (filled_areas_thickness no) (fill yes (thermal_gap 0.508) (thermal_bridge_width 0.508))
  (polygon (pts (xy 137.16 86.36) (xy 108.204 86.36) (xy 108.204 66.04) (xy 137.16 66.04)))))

